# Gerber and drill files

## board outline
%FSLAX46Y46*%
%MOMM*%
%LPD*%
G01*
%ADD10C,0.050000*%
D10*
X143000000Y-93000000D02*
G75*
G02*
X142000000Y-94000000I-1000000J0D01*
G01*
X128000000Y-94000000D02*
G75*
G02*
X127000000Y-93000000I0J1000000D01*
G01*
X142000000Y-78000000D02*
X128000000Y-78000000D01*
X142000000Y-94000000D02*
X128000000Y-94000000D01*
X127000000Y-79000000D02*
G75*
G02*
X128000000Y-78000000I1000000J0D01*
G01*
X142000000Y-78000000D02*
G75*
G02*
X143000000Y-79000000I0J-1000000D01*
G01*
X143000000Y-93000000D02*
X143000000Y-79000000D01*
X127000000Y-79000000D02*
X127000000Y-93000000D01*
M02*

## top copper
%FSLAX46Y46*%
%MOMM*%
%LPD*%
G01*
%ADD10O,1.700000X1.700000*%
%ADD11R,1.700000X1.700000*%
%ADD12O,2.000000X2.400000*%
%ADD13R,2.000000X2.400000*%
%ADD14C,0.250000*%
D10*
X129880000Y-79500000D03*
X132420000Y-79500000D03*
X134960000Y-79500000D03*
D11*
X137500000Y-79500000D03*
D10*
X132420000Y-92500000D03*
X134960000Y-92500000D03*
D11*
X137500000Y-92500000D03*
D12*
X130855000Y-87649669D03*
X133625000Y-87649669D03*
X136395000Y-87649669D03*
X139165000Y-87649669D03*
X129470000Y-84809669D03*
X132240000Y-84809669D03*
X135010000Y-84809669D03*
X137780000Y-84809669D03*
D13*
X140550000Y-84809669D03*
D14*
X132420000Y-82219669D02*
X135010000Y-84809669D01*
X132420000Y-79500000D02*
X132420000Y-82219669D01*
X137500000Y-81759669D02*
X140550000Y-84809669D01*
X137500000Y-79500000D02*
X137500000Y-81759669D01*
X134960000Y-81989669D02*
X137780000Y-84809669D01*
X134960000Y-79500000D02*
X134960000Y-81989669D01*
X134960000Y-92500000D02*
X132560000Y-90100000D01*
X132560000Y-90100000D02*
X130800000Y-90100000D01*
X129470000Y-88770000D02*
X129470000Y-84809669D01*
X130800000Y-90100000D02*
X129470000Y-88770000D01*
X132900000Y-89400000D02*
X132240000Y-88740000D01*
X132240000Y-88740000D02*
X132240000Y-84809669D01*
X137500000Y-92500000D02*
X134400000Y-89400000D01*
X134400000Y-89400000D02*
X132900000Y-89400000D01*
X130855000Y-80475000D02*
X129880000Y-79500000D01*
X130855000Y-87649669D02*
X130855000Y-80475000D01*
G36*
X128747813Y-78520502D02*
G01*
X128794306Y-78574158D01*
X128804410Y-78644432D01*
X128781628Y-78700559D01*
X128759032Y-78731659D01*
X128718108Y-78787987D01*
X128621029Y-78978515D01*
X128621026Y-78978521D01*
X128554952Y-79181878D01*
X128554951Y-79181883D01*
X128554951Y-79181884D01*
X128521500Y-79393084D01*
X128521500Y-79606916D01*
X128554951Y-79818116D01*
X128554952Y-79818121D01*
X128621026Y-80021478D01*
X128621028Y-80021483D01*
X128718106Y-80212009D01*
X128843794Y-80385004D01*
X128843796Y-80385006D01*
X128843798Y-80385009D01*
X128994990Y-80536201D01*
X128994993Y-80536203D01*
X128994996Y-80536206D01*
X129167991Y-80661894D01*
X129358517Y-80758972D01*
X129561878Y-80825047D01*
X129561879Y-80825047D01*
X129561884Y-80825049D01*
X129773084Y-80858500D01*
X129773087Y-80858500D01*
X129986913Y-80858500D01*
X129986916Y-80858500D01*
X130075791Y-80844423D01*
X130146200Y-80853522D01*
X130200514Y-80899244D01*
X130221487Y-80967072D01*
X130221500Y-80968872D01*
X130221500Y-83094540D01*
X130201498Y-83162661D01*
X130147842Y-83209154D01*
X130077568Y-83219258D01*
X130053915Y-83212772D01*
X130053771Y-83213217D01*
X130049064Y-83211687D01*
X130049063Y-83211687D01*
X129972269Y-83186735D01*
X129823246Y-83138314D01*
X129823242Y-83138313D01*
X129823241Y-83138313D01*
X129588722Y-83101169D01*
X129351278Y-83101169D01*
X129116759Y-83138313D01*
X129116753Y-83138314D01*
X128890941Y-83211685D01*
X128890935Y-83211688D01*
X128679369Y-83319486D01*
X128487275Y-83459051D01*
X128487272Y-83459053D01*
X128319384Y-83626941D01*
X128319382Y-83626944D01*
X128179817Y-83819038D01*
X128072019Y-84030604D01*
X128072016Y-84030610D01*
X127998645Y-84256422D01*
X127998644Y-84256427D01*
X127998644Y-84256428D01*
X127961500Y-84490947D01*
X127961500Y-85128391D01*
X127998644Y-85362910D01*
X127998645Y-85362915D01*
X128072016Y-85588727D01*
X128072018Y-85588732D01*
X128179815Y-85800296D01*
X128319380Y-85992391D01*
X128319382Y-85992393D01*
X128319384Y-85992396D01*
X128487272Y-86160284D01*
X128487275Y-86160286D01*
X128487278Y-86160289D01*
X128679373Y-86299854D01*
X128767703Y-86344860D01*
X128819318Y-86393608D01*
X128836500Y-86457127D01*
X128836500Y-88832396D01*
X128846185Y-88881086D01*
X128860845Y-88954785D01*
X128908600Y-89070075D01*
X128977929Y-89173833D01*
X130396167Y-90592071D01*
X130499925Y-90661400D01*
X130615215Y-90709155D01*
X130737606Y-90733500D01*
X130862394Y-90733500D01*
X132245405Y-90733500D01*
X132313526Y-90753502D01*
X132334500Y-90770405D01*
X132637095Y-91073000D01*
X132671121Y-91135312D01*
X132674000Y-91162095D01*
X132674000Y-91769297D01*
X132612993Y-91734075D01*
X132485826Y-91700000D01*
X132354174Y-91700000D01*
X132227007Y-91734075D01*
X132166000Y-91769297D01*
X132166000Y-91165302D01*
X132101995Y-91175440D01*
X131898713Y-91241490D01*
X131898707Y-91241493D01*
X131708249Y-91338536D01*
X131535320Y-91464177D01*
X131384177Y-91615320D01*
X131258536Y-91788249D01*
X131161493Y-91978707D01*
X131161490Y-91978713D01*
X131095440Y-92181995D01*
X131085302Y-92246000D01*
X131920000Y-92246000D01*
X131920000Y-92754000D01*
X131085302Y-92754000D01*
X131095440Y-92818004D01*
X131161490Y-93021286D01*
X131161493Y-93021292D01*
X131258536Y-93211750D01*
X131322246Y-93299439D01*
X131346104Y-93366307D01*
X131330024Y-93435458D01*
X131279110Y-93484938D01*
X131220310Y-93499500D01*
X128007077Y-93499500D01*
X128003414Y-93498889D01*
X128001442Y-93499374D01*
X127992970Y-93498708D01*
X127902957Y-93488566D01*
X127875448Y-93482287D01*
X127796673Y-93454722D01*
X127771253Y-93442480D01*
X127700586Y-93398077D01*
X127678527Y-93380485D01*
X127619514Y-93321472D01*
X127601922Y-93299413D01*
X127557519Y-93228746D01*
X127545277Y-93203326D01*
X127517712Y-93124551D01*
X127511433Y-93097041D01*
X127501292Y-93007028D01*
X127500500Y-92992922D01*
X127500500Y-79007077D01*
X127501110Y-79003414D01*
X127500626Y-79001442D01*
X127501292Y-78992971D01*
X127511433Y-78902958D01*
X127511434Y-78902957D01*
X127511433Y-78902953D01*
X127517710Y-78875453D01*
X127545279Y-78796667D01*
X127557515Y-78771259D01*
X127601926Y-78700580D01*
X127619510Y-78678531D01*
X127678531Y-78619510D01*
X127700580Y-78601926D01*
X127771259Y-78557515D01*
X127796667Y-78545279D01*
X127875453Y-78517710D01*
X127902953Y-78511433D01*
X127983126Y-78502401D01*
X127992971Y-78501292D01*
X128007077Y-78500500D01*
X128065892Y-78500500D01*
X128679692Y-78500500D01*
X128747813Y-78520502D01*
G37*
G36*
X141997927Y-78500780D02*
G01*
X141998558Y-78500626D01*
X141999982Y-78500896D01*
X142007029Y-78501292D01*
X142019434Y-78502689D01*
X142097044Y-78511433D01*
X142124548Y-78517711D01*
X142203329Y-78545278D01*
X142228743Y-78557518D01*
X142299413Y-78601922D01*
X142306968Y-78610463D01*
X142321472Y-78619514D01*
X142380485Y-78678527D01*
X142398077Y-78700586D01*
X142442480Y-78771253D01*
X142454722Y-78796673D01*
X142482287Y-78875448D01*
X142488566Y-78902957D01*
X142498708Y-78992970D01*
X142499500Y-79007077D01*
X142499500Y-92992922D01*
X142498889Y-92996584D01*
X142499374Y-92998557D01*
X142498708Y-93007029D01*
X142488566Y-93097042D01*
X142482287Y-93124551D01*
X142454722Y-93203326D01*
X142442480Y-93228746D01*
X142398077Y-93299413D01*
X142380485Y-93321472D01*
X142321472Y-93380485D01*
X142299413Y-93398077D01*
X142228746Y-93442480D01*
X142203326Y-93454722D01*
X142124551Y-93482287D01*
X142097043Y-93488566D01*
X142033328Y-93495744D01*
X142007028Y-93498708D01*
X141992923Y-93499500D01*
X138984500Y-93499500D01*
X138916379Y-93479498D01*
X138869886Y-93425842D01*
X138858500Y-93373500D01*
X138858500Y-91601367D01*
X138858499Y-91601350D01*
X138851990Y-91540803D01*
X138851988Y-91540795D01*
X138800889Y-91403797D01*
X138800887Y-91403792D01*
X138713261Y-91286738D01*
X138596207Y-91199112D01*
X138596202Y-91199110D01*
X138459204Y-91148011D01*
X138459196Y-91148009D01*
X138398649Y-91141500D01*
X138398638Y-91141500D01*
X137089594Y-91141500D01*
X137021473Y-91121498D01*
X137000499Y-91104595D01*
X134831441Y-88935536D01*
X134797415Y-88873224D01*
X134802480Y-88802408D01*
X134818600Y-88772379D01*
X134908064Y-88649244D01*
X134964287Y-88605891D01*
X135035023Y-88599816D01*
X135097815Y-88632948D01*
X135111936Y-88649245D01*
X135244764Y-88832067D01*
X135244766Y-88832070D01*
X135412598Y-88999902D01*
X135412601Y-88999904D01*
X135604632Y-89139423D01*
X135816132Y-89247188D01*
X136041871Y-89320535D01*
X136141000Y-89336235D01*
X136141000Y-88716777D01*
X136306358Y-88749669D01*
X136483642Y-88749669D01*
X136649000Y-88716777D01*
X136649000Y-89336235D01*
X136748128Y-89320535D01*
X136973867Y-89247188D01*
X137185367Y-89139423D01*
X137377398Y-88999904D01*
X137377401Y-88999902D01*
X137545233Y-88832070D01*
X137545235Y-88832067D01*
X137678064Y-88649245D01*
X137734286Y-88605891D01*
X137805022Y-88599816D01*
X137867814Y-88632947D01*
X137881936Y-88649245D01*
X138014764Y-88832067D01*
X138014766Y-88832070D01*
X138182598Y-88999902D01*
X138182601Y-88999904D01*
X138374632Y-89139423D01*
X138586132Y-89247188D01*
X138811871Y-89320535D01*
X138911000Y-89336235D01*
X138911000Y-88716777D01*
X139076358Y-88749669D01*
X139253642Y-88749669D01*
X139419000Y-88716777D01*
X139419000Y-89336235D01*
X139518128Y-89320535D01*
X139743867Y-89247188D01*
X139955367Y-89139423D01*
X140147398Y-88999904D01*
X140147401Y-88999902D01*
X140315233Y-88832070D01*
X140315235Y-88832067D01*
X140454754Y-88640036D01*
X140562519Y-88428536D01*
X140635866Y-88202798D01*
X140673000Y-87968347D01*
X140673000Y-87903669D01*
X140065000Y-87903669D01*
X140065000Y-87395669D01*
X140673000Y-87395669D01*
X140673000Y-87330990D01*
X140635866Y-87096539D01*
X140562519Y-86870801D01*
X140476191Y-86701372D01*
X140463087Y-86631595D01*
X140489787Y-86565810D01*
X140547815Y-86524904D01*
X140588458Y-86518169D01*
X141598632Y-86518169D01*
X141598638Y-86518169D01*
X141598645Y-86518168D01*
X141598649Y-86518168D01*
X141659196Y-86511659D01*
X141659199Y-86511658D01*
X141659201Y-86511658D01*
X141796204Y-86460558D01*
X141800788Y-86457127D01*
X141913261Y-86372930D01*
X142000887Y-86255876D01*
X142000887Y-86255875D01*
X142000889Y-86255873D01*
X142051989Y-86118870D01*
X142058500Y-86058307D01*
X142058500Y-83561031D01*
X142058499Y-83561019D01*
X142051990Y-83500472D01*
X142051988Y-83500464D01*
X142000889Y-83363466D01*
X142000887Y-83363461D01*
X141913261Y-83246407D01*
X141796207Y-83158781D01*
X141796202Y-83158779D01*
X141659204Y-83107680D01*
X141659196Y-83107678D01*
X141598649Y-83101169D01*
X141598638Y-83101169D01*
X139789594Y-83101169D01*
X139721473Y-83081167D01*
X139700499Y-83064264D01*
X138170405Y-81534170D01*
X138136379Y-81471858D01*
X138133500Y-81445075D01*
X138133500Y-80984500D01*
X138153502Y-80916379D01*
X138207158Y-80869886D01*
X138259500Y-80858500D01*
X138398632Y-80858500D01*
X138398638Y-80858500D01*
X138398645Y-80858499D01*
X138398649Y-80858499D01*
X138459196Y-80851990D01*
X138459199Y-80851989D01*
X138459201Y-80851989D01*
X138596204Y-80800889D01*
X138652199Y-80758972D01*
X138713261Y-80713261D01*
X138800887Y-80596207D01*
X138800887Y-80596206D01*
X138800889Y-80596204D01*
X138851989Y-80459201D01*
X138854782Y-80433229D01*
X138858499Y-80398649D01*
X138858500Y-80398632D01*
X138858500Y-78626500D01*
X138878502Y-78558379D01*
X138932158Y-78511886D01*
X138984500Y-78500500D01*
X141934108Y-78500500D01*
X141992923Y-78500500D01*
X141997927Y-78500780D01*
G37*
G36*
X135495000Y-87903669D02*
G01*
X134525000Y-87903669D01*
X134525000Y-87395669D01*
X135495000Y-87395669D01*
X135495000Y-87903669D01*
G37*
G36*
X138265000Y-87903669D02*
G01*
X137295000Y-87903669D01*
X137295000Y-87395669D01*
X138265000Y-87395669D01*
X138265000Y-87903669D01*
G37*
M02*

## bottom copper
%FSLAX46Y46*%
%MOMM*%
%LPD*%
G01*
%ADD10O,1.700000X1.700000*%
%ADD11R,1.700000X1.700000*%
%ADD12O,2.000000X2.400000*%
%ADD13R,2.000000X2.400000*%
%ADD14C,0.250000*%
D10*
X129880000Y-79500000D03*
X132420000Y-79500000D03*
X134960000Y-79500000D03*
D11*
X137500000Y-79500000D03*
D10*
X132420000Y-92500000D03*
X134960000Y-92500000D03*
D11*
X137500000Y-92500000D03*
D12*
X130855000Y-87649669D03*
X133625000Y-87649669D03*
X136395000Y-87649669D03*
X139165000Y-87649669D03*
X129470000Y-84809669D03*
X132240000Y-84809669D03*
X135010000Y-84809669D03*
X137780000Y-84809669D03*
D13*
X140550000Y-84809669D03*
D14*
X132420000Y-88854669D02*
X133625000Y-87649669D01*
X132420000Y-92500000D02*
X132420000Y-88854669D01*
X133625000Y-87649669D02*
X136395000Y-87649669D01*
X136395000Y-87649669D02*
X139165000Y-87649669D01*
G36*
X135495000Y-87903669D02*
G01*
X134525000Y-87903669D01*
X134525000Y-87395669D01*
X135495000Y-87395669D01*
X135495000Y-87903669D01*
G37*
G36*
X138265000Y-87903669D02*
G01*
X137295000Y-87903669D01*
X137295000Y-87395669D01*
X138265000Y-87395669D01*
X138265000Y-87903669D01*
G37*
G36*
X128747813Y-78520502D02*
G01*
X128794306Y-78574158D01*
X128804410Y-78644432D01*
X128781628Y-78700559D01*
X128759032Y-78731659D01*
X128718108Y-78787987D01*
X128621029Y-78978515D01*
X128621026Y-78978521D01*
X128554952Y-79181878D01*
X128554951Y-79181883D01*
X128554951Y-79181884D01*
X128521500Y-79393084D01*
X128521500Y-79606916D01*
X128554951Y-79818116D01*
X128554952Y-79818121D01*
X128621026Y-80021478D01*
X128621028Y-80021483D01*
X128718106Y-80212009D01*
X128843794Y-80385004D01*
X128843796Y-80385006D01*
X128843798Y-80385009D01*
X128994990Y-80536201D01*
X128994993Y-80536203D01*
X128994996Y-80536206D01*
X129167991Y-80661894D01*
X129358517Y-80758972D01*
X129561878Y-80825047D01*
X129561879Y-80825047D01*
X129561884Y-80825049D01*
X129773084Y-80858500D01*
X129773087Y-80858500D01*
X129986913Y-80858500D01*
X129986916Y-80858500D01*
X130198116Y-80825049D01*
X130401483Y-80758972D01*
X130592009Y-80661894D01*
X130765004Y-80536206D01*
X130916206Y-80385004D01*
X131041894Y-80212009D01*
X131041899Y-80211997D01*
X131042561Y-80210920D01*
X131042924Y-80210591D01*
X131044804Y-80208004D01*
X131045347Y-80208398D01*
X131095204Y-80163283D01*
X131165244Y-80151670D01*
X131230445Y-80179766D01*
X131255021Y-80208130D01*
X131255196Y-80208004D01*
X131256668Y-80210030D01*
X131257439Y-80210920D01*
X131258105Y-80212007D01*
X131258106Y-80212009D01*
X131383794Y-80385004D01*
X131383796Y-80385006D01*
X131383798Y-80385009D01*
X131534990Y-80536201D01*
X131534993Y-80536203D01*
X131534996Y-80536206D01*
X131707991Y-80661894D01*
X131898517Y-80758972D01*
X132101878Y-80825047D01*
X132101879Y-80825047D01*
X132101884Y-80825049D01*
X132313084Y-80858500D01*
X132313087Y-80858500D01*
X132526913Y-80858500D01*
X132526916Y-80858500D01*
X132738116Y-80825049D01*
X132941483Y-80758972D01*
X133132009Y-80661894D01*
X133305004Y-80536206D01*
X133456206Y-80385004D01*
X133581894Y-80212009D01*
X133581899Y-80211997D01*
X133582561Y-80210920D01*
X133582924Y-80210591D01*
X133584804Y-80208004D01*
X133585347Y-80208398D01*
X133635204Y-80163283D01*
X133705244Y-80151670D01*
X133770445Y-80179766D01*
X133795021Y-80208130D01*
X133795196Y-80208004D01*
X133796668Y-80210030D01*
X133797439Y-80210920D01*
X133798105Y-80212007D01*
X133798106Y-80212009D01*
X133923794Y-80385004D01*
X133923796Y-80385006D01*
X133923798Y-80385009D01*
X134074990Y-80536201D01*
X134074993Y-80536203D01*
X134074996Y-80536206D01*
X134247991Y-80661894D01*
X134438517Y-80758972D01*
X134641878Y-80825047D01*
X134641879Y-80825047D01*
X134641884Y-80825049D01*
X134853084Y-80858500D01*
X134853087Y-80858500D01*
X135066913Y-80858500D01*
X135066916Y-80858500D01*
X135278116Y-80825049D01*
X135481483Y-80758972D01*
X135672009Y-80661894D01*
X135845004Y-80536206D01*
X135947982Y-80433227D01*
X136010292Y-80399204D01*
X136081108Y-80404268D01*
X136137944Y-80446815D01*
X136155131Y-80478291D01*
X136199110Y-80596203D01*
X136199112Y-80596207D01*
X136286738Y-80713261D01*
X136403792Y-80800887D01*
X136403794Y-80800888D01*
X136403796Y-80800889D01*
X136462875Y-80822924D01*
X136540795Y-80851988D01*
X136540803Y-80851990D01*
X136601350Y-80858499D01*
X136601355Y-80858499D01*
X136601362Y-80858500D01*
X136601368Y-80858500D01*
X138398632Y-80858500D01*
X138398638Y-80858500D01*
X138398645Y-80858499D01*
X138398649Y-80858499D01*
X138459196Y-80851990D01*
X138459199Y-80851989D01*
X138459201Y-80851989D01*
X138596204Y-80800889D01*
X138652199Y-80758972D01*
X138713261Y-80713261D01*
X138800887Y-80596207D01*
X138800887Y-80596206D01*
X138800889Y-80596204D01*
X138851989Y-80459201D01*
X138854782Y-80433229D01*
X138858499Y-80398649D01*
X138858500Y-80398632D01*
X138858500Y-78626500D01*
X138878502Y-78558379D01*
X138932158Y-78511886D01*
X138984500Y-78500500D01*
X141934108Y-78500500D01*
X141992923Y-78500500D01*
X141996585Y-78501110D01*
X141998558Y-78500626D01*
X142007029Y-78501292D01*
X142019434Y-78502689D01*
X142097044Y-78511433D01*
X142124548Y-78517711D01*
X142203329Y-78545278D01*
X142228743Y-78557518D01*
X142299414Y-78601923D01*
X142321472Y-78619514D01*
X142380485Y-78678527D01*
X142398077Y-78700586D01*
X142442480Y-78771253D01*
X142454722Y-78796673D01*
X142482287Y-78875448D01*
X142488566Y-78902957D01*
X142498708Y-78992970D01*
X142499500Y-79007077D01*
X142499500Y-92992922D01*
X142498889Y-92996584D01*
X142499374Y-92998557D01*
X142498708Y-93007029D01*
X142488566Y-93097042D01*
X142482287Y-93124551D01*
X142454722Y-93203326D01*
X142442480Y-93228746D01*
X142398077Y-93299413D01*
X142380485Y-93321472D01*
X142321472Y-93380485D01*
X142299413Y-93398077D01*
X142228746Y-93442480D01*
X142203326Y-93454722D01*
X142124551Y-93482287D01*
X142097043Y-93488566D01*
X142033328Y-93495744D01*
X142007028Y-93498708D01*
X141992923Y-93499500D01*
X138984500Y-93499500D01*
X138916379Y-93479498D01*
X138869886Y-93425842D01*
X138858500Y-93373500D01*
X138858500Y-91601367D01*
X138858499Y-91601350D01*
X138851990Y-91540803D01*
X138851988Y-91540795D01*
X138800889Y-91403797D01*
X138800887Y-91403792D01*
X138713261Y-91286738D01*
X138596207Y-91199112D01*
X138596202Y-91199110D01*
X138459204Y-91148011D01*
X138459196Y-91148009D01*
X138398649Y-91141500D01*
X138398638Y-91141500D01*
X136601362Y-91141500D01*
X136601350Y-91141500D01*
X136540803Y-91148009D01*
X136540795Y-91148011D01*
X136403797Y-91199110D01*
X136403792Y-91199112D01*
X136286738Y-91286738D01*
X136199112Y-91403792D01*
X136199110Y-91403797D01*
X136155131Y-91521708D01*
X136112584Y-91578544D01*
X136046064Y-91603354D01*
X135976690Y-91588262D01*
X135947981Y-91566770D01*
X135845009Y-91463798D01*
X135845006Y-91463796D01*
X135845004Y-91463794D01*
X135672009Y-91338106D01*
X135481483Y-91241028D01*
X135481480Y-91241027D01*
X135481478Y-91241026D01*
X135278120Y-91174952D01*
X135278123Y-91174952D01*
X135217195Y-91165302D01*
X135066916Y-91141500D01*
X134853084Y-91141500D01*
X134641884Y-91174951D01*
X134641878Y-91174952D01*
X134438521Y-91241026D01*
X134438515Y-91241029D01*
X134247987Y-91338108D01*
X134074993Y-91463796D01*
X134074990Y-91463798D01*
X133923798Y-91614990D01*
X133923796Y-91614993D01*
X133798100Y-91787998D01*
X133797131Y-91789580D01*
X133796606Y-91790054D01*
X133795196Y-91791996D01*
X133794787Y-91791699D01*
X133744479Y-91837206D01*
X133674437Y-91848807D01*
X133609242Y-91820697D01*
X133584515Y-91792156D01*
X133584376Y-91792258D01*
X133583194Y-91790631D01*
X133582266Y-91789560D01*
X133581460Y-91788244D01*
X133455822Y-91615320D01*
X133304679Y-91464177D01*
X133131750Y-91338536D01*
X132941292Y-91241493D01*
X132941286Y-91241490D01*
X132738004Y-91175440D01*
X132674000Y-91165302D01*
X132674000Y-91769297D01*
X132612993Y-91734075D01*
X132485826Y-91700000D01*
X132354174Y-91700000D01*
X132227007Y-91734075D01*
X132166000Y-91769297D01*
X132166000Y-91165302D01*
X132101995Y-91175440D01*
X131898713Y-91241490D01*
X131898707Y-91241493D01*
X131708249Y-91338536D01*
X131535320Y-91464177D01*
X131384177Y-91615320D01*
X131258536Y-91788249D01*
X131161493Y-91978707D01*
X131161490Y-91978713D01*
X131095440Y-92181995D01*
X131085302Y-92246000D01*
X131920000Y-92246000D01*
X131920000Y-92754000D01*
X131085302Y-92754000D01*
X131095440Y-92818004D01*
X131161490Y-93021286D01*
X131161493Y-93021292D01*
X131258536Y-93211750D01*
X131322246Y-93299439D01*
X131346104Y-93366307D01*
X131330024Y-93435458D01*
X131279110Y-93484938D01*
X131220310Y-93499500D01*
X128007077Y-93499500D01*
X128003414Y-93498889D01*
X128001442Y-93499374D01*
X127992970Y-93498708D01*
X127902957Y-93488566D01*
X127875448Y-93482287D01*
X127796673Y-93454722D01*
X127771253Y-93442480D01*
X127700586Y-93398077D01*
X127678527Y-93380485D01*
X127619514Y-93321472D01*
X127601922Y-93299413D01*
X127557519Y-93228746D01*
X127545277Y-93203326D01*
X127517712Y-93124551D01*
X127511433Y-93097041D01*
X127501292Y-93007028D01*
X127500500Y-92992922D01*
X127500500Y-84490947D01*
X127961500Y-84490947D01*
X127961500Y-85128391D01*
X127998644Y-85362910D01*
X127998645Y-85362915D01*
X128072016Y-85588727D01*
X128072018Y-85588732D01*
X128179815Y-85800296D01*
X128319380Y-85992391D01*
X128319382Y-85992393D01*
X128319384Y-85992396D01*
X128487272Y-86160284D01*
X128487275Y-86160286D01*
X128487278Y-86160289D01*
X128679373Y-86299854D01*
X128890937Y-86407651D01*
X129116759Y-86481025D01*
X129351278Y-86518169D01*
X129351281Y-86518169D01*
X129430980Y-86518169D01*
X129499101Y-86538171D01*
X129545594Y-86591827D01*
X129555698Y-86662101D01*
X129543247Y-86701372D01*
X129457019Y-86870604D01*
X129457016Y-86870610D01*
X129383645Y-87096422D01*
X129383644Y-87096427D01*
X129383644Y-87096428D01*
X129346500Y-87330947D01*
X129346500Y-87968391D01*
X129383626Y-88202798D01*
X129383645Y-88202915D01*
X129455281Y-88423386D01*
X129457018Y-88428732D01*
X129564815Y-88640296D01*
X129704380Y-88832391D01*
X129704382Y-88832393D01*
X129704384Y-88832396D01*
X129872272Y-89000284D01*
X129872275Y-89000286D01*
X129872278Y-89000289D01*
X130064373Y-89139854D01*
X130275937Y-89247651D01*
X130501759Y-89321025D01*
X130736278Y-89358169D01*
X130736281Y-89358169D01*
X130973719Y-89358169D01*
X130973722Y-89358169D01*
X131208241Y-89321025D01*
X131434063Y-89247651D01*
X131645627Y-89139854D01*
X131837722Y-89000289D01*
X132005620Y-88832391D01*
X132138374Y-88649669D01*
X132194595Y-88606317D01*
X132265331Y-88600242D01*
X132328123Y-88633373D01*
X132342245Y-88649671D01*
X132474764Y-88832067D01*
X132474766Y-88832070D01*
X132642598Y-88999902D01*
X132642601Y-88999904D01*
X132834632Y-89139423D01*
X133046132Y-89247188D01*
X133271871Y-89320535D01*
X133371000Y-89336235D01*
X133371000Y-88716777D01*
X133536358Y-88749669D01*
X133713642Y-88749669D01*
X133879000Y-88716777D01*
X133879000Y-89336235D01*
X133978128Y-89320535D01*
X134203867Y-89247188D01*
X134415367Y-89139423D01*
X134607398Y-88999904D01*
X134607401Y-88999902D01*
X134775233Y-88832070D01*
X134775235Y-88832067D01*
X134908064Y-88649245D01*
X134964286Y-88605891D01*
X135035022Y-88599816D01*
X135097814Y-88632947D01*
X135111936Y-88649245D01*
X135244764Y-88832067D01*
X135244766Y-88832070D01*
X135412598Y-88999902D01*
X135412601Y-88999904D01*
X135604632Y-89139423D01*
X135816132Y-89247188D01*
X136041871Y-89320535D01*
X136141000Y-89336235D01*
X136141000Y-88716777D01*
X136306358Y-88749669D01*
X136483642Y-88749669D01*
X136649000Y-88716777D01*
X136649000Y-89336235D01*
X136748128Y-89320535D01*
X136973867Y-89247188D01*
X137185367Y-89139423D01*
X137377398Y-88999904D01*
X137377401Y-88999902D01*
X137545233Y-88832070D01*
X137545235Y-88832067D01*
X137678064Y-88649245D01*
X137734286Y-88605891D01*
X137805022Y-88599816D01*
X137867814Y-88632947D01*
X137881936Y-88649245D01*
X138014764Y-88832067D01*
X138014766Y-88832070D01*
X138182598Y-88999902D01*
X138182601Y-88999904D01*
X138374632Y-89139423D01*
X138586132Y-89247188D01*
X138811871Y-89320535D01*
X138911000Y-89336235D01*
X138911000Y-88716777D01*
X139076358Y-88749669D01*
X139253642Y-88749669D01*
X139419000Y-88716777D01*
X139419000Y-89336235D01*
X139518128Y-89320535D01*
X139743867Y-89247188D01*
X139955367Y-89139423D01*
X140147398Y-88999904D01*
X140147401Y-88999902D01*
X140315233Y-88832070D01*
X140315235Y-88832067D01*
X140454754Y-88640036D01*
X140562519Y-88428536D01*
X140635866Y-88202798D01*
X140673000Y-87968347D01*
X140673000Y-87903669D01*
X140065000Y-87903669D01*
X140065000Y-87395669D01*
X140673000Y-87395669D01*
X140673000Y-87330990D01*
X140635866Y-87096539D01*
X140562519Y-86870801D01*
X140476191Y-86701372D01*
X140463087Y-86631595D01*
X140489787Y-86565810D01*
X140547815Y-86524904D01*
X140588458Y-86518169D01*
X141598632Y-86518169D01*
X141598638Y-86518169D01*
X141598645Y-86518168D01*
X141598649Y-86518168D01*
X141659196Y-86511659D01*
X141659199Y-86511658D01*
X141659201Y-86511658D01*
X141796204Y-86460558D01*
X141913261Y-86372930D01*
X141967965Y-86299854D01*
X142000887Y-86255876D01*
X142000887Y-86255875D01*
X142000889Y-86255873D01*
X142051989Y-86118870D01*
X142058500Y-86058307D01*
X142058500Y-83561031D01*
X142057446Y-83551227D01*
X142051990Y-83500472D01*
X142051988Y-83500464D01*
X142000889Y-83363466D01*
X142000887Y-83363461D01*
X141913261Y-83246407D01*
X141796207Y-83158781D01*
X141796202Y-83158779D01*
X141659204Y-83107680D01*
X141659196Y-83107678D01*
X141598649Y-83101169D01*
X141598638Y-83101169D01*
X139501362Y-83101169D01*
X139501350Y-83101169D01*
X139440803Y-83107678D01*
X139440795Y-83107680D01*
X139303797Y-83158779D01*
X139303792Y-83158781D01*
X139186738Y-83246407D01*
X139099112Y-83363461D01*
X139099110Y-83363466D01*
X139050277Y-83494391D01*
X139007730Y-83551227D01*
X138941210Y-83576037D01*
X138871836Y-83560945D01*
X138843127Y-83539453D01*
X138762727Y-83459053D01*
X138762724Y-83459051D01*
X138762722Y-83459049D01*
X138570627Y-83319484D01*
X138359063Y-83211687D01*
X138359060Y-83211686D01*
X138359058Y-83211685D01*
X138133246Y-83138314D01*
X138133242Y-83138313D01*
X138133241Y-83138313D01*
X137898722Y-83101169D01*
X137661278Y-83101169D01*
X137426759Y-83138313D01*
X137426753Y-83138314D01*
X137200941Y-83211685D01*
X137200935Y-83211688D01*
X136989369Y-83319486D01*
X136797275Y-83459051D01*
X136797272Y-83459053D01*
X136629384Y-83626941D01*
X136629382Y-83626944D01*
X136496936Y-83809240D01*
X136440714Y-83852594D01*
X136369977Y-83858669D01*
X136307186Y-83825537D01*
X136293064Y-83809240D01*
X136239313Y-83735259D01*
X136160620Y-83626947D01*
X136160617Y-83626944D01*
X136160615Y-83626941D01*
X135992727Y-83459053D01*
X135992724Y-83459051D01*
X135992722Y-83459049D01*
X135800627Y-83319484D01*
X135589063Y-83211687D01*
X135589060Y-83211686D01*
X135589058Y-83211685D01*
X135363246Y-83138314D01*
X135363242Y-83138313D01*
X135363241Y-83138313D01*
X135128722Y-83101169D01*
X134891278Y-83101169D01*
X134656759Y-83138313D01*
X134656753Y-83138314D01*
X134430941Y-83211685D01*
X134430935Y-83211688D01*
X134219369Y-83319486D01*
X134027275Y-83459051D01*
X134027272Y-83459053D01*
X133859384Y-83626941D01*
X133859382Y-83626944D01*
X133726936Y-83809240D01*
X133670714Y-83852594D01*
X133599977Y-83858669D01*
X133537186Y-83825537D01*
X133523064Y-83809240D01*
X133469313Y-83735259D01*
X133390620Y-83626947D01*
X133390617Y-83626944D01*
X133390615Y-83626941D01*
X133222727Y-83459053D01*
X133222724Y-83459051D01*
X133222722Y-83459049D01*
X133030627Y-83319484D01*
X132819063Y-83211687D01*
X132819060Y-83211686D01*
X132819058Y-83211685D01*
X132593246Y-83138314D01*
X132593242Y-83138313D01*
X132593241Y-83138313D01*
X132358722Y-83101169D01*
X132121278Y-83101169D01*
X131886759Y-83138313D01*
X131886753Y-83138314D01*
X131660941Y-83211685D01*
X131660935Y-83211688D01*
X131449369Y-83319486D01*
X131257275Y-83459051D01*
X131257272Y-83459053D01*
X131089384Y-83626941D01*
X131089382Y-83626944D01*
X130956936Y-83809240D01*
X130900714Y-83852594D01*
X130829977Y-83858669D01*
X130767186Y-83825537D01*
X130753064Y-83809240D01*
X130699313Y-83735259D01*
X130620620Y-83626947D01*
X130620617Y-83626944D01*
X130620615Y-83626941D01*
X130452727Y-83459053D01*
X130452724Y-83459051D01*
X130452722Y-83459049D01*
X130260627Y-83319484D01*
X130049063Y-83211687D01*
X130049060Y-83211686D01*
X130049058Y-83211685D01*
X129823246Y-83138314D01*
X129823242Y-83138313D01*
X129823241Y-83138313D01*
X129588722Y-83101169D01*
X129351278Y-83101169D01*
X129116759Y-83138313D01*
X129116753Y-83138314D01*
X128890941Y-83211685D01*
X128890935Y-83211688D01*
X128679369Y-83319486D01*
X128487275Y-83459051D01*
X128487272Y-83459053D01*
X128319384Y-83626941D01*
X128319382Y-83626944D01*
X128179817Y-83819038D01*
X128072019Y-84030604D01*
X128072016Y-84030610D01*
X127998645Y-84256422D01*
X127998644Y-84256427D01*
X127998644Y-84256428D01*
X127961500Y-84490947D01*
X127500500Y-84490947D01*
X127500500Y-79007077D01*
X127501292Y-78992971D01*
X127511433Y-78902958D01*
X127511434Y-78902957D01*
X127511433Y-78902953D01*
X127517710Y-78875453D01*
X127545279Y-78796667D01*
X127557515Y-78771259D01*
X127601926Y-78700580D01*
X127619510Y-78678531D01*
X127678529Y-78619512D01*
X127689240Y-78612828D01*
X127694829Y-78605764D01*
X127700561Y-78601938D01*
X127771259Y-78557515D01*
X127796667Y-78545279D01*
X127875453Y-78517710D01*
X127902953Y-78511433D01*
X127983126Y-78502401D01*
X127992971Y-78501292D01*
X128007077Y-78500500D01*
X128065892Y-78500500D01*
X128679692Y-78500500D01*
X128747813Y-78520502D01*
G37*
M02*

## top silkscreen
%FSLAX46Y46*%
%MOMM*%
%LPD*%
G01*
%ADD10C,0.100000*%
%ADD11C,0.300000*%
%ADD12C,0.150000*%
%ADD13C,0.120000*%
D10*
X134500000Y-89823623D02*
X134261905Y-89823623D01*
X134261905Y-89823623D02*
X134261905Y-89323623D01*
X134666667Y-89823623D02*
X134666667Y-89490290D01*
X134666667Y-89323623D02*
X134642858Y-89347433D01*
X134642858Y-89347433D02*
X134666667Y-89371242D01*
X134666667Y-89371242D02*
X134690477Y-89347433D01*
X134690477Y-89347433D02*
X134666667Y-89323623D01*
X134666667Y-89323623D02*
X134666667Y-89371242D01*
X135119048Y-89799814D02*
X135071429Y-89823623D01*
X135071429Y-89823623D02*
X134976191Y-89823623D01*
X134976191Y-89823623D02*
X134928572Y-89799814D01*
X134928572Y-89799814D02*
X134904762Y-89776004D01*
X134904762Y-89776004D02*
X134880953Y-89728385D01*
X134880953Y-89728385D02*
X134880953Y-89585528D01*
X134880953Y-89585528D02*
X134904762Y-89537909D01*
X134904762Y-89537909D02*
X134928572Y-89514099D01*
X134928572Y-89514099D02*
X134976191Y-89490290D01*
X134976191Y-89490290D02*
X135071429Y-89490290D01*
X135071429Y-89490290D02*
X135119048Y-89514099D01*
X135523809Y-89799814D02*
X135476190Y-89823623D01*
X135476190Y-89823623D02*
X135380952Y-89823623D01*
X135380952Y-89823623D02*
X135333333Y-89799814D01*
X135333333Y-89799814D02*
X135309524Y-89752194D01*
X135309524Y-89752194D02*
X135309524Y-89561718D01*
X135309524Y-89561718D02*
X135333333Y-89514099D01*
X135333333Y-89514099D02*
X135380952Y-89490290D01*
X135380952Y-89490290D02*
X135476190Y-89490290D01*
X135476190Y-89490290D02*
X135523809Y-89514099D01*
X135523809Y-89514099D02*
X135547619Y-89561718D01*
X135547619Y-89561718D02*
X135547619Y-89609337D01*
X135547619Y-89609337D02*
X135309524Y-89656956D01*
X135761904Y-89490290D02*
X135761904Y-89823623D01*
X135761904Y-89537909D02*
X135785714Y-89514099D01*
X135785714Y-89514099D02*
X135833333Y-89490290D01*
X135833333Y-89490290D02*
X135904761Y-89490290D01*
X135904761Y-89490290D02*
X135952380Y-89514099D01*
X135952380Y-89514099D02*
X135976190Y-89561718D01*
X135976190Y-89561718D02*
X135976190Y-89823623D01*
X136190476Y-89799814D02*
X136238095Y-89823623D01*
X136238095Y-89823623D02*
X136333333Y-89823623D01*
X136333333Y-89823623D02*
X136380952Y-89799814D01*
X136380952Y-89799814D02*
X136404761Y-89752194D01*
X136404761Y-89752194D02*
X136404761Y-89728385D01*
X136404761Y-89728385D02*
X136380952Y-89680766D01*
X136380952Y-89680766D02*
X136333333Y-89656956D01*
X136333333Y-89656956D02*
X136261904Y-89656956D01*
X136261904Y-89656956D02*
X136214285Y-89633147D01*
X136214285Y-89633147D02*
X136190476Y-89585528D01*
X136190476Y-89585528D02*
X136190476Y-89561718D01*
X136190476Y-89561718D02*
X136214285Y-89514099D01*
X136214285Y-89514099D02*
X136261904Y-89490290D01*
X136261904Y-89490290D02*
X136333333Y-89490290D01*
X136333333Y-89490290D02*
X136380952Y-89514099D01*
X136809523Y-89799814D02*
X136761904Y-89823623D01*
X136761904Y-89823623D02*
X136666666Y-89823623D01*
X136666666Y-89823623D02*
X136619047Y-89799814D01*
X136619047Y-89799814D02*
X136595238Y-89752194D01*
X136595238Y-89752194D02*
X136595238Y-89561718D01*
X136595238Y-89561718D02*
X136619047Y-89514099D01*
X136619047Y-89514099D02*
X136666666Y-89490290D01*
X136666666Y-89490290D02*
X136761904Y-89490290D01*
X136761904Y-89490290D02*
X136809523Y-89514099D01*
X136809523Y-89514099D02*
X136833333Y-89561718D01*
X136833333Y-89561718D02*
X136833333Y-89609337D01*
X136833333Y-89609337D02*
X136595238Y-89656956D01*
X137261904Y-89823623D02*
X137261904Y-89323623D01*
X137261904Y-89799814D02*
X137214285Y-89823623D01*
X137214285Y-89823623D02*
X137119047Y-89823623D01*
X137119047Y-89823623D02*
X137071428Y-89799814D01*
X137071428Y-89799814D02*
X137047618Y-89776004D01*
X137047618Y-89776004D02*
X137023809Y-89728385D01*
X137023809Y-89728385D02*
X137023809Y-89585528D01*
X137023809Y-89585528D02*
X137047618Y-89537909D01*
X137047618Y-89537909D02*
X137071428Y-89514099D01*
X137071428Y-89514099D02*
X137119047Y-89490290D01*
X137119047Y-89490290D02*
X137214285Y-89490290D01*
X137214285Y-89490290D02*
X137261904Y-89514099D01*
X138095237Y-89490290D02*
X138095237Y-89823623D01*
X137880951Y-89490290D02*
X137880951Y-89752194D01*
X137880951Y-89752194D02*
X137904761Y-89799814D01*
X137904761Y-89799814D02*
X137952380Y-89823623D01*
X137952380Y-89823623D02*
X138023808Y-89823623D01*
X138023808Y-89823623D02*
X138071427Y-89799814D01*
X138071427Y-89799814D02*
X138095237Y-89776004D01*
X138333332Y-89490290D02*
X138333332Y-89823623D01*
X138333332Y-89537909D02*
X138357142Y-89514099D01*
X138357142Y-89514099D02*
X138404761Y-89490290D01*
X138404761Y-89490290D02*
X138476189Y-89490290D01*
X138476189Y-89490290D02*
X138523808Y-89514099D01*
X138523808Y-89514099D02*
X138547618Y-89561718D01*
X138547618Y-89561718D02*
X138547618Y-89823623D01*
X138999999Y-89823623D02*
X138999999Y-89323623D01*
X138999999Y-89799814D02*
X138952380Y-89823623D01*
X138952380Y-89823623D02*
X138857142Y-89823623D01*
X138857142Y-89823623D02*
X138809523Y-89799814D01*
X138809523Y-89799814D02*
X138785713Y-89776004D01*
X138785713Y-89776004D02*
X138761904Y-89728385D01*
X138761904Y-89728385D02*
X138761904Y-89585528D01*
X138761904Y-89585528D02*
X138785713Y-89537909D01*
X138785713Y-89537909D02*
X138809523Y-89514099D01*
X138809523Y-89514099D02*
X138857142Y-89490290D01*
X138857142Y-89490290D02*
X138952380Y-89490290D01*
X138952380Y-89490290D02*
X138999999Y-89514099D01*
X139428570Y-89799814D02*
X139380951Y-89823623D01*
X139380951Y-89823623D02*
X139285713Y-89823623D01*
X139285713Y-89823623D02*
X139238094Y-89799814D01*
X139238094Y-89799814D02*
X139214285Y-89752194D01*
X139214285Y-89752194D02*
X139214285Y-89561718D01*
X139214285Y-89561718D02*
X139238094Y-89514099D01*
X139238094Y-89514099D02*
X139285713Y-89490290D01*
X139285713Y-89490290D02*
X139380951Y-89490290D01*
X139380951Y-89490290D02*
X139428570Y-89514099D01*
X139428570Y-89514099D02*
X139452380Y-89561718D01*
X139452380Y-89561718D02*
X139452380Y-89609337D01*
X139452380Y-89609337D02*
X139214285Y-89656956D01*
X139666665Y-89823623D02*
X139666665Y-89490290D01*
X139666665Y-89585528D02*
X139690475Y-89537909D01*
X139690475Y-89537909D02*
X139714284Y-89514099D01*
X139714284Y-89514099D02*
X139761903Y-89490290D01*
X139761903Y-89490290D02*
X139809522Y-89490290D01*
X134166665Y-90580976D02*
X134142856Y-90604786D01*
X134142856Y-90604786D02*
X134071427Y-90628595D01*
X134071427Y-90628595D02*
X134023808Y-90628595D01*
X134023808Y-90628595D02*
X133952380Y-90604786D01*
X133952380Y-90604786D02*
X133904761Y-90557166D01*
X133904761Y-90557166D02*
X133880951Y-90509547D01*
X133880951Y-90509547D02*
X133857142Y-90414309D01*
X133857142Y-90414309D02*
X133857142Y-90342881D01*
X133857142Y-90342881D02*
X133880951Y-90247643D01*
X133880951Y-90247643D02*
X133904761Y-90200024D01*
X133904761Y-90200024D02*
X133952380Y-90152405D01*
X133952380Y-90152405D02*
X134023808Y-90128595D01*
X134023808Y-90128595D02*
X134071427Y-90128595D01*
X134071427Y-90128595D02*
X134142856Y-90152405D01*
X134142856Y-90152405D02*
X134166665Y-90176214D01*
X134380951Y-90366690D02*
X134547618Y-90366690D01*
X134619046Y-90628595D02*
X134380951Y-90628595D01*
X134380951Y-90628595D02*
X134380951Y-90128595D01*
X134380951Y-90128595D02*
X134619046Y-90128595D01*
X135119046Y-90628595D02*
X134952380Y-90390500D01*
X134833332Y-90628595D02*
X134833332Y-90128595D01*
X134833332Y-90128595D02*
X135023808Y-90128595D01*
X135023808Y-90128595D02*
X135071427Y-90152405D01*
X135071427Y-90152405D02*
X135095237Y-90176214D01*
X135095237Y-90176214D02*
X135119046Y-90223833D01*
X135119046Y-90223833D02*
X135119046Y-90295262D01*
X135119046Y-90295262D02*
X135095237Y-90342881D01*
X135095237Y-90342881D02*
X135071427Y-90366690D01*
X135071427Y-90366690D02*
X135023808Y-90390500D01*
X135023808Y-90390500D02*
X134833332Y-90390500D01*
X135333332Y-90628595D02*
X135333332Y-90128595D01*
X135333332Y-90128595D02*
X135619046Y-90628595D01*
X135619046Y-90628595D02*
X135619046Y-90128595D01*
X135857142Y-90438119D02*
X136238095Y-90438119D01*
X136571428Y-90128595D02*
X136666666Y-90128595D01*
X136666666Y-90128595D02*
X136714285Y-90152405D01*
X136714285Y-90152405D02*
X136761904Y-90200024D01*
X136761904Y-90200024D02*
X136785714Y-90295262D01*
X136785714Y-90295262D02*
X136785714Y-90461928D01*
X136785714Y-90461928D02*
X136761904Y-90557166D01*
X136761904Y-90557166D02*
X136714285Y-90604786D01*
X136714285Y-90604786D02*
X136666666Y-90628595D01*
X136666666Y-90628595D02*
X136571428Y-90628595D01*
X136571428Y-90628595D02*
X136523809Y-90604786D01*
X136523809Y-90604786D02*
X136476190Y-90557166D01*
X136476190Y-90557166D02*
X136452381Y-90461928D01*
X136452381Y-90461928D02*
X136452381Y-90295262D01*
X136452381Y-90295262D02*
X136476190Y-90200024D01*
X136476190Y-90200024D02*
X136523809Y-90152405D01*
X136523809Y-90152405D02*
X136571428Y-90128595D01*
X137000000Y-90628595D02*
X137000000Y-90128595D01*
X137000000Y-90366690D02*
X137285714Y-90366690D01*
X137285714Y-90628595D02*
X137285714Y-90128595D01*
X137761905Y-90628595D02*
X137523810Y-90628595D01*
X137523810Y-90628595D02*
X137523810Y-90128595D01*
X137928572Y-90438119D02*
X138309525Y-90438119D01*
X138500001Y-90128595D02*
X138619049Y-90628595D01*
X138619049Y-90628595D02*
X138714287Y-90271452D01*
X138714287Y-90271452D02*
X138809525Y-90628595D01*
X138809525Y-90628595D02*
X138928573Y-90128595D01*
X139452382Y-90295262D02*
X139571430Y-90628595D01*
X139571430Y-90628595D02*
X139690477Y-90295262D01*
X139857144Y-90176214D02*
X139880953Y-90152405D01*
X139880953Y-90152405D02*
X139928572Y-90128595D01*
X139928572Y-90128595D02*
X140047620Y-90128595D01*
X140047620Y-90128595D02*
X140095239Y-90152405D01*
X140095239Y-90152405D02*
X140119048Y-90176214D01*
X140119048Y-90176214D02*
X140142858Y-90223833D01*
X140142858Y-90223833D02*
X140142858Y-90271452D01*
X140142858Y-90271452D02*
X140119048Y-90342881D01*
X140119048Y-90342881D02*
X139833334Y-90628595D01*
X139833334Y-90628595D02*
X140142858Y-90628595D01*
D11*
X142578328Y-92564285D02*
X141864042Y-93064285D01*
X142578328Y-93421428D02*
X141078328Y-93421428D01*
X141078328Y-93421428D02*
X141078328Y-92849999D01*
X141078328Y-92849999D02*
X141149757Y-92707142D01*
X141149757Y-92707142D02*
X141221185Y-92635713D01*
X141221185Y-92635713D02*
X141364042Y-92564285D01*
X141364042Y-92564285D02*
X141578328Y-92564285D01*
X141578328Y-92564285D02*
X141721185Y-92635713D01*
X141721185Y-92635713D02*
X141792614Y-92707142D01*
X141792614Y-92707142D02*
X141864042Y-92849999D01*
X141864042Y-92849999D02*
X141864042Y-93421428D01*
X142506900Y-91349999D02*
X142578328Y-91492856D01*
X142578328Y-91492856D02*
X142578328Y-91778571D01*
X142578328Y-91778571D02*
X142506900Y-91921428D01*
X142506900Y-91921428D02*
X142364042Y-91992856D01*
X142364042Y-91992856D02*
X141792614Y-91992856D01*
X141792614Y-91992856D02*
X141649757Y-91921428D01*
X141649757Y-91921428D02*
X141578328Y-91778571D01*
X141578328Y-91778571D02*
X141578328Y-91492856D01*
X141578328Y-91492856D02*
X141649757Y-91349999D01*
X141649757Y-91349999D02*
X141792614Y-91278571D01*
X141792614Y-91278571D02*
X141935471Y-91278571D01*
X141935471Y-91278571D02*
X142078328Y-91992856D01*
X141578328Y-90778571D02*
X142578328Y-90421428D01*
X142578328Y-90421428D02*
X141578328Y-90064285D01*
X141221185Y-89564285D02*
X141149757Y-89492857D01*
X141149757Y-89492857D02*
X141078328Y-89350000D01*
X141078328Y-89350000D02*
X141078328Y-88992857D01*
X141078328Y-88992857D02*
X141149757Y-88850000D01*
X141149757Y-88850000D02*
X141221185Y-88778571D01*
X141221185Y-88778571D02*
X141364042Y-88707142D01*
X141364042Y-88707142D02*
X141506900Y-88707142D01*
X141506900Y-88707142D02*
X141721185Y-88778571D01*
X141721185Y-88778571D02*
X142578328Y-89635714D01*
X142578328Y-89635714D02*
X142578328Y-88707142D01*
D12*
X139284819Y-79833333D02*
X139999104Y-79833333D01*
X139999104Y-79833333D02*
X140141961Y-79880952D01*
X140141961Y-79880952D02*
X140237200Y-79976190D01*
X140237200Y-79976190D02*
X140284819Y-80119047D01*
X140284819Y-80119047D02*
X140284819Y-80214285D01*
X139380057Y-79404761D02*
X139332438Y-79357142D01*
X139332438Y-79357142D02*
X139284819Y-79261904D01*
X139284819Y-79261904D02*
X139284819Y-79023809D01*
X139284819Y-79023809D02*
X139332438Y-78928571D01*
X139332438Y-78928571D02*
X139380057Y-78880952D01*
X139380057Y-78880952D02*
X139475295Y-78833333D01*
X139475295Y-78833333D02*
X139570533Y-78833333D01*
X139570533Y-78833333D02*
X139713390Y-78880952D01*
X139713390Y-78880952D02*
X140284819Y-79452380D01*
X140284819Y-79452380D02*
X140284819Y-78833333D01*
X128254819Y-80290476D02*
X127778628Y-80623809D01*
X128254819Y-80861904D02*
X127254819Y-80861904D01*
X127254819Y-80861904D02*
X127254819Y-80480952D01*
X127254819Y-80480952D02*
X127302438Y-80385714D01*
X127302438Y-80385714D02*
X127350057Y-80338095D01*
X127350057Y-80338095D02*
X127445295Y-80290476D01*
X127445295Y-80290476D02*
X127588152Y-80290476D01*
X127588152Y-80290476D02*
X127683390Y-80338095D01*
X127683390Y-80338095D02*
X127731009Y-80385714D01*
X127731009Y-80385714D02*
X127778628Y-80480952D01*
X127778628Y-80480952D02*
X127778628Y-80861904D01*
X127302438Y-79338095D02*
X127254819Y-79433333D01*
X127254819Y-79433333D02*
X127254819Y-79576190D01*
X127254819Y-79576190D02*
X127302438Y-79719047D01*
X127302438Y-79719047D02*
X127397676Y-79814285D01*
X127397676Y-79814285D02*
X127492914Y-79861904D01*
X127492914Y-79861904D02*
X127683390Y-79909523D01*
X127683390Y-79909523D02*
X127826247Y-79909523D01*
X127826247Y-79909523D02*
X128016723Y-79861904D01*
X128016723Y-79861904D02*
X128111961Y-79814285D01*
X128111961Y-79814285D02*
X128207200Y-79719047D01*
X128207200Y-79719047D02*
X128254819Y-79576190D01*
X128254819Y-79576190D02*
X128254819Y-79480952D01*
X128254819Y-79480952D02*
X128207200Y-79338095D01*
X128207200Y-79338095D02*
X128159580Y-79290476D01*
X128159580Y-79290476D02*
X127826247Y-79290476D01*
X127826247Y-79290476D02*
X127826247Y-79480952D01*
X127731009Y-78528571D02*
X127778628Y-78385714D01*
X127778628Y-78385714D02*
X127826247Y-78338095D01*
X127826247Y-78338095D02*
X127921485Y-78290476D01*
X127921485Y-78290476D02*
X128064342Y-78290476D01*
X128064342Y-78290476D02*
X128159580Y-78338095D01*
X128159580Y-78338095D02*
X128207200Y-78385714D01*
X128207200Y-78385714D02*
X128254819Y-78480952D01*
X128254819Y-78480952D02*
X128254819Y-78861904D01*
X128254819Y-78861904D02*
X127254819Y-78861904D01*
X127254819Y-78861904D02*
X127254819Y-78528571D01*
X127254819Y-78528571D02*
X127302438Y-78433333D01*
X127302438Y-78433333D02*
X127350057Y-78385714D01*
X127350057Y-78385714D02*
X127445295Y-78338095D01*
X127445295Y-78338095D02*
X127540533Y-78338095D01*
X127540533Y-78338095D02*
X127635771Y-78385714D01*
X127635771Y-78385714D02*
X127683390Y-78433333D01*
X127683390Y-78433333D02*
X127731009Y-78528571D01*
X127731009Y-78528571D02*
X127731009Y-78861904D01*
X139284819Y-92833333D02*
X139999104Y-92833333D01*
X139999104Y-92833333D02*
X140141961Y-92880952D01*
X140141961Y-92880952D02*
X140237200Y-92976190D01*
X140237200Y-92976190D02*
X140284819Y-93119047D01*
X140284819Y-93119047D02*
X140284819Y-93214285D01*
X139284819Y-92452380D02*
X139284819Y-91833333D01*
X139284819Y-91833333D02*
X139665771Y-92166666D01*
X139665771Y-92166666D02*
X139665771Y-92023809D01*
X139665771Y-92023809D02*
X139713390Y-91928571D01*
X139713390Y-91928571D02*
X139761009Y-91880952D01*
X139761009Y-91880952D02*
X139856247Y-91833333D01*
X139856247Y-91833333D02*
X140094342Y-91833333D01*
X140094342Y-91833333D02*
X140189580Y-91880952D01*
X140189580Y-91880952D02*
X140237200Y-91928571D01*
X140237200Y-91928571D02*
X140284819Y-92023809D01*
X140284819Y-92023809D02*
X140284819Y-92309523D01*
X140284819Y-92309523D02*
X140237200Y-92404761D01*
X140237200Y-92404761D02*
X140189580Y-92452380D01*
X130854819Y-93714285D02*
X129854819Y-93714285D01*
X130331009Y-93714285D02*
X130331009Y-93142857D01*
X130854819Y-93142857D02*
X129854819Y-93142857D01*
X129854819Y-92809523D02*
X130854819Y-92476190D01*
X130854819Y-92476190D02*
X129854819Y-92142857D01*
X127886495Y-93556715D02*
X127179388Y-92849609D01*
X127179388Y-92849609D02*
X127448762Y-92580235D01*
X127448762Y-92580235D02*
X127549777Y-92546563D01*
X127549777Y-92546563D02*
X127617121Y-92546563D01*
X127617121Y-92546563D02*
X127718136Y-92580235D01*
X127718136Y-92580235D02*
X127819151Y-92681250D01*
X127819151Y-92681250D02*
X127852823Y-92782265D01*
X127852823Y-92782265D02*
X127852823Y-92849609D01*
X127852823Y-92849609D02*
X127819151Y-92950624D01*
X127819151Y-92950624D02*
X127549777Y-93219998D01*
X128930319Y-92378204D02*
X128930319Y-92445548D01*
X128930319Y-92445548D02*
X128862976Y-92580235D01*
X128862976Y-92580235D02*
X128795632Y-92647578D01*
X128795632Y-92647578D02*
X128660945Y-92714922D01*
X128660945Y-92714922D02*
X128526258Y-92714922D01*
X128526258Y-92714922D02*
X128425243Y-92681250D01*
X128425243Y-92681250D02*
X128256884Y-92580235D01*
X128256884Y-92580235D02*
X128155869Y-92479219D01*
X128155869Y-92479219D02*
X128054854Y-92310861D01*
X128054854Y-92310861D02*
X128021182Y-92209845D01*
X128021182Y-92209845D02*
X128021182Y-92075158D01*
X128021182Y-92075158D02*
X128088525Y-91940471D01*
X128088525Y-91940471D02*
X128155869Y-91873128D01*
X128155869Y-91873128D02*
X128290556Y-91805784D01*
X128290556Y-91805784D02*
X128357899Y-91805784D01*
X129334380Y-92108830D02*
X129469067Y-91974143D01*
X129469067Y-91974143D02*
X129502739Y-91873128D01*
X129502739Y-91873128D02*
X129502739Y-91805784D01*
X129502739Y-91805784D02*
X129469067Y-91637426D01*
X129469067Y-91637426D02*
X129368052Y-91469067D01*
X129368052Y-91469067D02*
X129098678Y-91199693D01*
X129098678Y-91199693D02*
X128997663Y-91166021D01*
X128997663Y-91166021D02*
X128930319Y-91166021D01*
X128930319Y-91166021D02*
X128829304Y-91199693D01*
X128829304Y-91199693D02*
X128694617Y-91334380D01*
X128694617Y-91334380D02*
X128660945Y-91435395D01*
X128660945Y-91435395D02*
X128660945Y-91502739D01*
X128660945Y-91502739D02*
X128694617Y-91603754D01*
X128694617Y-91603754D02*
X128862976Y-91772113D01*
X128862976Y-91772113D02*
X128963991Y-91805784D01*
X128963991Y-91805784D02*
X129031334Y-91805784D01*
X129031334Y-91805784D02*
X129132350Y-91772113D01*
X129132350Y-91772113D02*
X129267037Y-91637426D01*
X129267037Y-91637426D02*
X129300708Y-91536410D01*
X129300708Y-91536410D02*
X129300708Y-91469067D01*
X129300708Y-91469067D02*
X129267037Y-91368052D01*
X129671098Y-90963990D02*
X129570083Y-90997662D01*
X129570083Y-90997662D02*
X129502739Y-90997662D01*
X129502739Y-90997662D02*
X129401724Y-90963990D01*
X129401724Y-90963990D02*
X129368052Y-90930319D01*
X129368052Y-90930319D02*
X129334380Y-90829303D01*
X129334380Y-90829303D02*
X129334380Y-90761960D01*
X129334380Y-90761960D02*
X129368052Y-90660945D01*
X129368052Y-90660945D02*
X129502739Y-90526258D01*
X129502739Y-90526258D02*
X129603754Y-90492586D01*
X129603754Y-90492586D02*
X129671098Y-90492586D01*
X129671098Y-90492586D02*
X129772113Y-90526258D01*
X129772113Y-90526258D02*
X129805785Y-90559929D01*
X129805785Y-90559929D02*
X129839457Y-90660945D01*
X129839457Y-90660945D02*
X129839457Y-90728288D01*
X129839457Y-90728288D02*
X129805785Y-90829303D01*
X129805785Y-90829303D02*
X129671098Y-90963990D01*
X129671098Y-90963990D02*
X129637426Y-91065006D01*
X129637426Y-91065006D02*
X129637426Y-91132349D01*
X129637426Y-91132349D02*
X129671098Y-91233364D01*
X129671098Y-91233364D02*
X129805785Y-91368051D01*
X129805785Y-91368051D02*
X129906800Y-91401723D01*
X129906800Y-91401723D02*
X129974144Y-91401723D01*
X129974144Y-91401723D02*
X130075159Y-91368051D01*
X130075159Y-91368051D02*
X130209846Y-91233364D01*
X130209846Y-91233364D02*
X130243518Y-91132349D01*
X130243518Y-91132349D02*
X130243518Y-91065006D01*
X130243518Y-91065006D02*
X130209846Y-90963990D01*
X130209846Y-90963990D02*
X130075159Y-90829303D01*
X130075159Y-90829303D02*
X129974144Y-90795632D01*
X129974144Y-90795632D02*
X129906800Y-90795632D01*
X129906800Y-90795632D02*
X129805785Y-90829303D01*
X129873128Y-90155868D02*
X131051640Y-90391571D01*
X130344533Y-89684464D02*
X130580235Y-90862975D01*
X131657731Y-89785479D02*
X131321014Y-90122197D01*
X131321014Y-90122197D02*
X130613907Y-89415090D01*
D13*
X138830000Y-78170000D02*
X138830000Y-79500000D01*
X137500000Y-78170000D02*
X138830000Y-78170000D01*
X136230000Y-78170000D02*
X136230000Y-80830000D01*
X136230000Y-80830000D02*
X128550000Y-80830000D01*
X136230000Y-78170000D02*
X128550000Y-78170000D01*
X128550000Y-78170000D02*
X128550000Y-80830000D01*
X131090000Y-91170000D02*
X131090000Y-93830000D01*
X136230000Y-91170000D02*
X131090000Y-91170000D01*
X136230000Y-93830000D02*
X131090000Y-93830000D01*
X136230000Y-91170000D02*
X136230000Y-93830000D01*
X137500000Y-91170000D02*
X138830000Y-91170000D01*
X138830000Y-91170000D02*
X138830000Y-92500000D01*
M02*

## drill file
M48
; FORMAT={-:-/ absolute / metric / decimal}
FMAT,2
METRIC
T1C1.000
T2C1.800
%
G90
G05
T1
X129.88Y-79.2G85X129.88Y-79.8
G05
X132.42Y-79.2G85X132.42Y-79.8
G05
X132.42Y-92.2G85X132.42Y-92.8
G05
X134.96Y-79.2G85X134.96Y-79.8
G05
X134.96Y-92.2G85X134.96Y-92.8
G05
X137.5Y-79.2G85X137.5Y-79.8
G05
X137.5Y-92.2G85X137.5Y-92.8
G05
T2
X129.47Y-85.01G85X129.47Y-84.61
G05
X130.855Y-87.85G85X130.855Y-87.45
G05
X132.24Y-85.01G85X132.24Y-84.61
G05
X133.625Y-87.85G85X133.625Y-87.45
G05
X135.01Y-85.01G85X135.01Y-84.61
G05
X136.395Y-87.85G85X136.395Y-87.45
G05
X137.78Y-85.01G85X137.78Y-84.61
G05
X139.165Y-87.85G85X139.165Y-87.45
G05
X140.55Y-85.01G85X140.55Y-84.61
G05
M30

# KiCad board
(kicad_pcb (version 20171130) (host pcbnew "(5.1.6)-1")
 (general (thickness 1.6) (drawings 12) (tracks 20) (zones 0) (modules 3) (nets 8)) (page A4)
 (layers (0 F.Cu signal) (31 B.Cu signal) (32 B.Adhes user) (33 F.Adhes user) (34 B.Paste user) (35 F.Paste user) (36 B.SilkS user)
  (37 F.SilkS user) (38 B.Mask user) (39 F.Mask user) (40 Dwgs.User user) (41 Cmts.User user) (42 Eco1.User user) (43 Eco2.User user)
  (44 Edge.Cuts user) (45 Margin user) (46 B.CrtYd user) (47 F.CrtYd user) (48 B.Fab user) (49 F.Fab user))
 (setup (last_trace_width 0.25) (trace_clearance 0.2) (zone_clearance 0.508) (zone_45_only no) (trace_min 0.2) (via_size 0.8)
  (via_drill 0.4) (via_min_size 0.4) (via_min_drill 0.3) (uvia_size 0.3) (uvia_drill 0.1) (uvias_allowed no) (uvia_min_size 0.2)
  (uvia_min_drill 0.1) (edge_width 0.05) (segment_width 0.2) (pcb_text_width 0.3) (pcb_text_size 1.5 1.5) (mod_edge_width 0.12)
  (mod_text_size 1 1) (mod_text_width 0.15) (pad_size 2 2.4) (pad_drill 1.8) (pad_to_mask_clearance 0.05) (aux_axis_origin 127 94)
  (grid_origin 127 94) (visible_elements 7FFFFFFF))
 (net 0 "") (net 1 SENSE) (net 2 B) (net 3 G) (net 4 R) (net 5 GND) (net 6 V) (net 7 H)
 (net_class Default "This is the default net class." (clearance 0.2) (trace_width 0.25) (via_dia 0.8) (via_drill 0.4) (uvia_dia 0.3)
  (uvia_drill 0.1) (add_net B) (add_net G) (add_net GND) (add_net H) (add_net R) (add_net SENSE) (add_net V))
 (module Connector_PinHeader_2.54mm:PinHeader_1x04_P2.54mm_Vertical (layer F.Cu) (at 137.5 79.5 270)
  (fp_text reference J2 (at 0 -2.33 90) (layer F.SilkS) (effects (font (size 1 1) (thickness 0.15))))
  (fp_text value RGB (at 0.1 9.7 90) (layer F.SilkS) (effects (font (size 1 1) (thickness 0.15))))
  (fp_line (start -1.33 -1.33) (end 0 -1.33) (layer F.SilkS) (width 0.12))
  (fp_line (start -1.33 0) (end -1.33 -1.33) (layer F.SilkS) (width 0.12))
  (fp_line (start -1.33 1.27) (end 1.33 1.27) (layer F.SilkS) (width 0.12))
  (fp_line (start 1.33 1.27) (end 1.33 8.95) (layer F.SilkS) (width 0.12))
  (fp_line (start -1.33 1.27) (end -1.33 8.95) (layer F.SilkS) (width 0.12))
  (fp_line (start -1.33 8.95) (end 1.33 8.95) (layer F.SilkS) (width 0.12))
  (pad 4 thru_hole oval (at 0 7.62 270) (size 1.7 1.7) (drill oval 1.6 1) (layers *.Cu *.Mask) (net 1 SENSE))
  (pad 3 thru_hole oval (at 0 5.08 270) (size 1.7 1.7) (drill oval 1.6 1) (layers *.Cu *.Mask) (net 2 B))
  (pad 2 thru_hole oval (at 0 2.54 270) (size 1.7 1.7) (drill oval 1.6 1) (layers *.Cu *.Mask) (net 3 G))
  (pad 1 thru_hole rect (at 0 0 270) (size 1.7 1.7) (drill oval 1.6 1) (layers *.Cu *.Mask) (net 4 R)))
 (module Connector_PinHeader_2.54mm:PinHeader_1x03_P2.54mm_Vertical (layer F.Cu) (at 137.5 92.5 270)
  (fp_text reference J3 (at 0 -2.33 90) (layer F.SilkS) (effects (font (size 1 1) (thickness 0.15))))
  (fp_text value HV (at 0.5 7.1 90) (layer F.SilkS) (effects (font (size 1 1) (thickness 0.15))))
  (fp_line (start -1.33 6.41) (end 1.33 6.41) (layer F.SilkS) (width 0.12))
  (fp_line (start -1.33 1.27) (end -1.33 6.41) (layer F.SilkS) (width 0.12))
  (fp_line (start 1.33 1.27) (end 1.33 6.41) (layer F.SilkS) (width 0.12))
  (fp_line (start -1.33 1.27) (end 1.33 1.27) (layer F.SilkS) (width 0.12))
  (fp_line (start -1.33 0) (end -1.33 -1.33) (layer F.SilkS) (width 0.12))
  (fp_line (start -1.33 -1.33) (end 0 -1.33) (layer F.SilkS) (width 0.12))
  (pad 3 thru_hole oval (at 0 5.08 270) (size 1.7 1.7) (drill oval 1.6 1) (layers *.Cu *.Mask) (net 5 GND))
  (pad 2 thru_hole oval (at 0 2.54 270) (size 1.7 1.7) (drill oval 1.6 1) (layers *.Cu *.Mask) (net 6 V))
  (pad 1 thru_hole rect (at 0 0 270) (size 1.7 1.7) (drill oval 1.6 1) (layers *.Cu *.Mask) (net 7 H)))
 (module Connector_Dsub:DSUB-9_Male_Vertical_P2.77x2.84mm (layer B.Cu) (at 140.55 84.809669 180)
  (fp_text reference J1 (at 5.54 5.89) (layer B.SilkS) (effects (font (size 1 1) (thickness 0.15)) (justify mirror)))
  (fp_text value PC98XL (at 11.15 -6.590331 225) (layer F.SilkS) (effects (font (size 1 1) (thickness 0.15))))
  (pad 9 thru_hole oval (at 9.695 -2.84 180) (size 2 2.4) (drill oval 1.8 2.2) (layers *.Cu *.Mask) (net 1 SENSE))
  (pad 8 thru_hole oval (at 6.925 -2.84 180) (size 2 2.4) (drill oval 1.8 2.2) (layers *.Cu *.Mask) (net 5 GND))
  (pad 7 thru_hole oval (at 4.155 -2.84 180) (size 2 2.4) (drill oval 1.8 2.2) (layers *.Cu *.Mask) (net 5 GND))
  (pad 6 thru_hole oval (at 1.385 -2.84 180) (size 2 2.4) (drill oval 1.8 2.2) (layers *.Cu *.Mask) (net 5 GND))
  (pad 5 thru_hole oval (at 11.08 0 180) (size 2 2.4) (drill oval 1.8 2.2) (layers *.Cu *.Mask) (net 6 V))
  (pad 4 thru_hole oval (at 8.31 0 180) (size 2 2.4) (drill oval 1.8 2.2) (layers *.Cu *.Mask) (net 7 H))
  (pad 3 thru_hole oval (at 5.54 0 180) (size 2 2.4) (drill oval 1.8 2.2) (layers *.Cu *.Mask) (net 2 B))
  (pad 2 thru_hole oval (at 2.77 0 180) (size 2 2.4) (drill oval 1.8 2.2) (layers *.Cu *.Mask) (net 3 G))
  (pad 1 thru_hole rect (at 0 0 180) (size 2 2.4) (drill oval 1.8 2.2) (layers *.Cu *.Mask) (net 4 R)))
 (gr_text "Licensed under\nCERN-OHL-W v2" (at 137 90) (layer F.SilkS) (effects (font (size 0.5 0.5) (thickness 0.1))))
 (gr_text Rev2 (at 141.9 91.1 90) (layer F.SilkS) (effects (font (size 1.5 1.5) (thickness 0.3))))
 (gr_arc (start 142 93) (end 142 94) (angle -90) (layer Edge.Cuts) (width 0.05))
 (gr_arc (start 128 93) (end 127 93) (angle -90) (layer Edge.Cuts) (width 0.05))
 (gr_line (start 142 78) (end 128 78) (layer Edge.Cuts) (width 0.05))
 (gr_line (start 142 94) (end 128 94) (layer Edge.Cuts) (width 0.05))
 (gr_arc (start 128 79) (end 128 78) (angle -90) (layer Edge.Cuts) (width 0.05))
 (gr_arc (start 142 79) (end 143 79) (angle -90) (layer Edge.Cuts) (width 0.05))
 (gr_line (start 143 93) (end 143 79) (layer Edge.Cuts) (width 0.05))
 (gr_line (start 127 79) (end 127 93) (layer Edge.Cuts) (width 0.05))
 (segment (start 132.42 82.219669) (end 135.01 84.809669) (width 0.25) (layer F.Cu) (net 2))
 (segment (start 132.42 79.5) (end 132.42 82.219669) (width 0.25) (layer F.Cu) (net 2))
 (segment (start 137.5 81.759669) (end 140.55 84.809669) (width 0.25) (layer F.Cu) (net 4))
 (segment (start 137.5 79.5) (end 137.5 81.759669) (width 0.25) (layer F.Cu) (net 4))
 (segment (start 134.96 81.989669) (end 137.78 84.809669) (width 0.25) (layer F.Cu) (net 3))
 (segment (start 134.96 79.5) (end 134.96 81.989669) (width 0.25) (layer F.Cu) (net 3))
 (segment (start 134.96 92.5) (end 132.56 90.1) (width 0.25) (layer F.Cu) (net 6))
 (segment (start 132.56 90.1) (end 130.8 90.1) (width 0.25) (layer F.Cu) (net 6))
 (segment (start 129.47 88.77) (end 129.47 84.809669) (width 0.25) (layer F.Cu) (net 6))
 (segment (start 130.8 90.1) (end 129.47 88.77) (width 0.25) (layer F.Cu) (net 6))
 (segment (start 132.9 89.4) (end 132.24 88.74) (width 0.25) (layer F.Cu) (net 7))
 (segment (start 132.24 88.74) (end 132.24 84.809669) (width 0.25) (layer F.Cu) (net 7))
 (segment (start 137.5 92.5) (end 134.4 89.4) (width 0.25) (layer F.Cu) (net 7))
 (segment (start 134.4 89.4) (end 132.9 89.4) (width 0.25) (layer F.Cu) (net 7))
 (segment (start 132.42 88.854669) (end 133.625 87.649669) (width 0.25) (layer B.Cu) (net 5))
 (segment (start 132.42 92.5) (end 132.42 88.854669) (width 0.25) (layer B.Cu) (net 5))
 (segment (start 133.625 87.649669) (end 136.395 87.649669) (width 0.25) (layer B.Cu) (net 5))
 (segment (start 136.395 87.649669) (end 139.165 87.649669) (width 0.25) (layer B.Cu) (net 5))
 (segment (start 130.855 80.475) (end 129.88 79.5) (width 0.25) (layer F.Cu) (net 1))
 (segment (start 130.855 87.649669) (end 130.855 80.475) (width 0.25) (layer F.Cu) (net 1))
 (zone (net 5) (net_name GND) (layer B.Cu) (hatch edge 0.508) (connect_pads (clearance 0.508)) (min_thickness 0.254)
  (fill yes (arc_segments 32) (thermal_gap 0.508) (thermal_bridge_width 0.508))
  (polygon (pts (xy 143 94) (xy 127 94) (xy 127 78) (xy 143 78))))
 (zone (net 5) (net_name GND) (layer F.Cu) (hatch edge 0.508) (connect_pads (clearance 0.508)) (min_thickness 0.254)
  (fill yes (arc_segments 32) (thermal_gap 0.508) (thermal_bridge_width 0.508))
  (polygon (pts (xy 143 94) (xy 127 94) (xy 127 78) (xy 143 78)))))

